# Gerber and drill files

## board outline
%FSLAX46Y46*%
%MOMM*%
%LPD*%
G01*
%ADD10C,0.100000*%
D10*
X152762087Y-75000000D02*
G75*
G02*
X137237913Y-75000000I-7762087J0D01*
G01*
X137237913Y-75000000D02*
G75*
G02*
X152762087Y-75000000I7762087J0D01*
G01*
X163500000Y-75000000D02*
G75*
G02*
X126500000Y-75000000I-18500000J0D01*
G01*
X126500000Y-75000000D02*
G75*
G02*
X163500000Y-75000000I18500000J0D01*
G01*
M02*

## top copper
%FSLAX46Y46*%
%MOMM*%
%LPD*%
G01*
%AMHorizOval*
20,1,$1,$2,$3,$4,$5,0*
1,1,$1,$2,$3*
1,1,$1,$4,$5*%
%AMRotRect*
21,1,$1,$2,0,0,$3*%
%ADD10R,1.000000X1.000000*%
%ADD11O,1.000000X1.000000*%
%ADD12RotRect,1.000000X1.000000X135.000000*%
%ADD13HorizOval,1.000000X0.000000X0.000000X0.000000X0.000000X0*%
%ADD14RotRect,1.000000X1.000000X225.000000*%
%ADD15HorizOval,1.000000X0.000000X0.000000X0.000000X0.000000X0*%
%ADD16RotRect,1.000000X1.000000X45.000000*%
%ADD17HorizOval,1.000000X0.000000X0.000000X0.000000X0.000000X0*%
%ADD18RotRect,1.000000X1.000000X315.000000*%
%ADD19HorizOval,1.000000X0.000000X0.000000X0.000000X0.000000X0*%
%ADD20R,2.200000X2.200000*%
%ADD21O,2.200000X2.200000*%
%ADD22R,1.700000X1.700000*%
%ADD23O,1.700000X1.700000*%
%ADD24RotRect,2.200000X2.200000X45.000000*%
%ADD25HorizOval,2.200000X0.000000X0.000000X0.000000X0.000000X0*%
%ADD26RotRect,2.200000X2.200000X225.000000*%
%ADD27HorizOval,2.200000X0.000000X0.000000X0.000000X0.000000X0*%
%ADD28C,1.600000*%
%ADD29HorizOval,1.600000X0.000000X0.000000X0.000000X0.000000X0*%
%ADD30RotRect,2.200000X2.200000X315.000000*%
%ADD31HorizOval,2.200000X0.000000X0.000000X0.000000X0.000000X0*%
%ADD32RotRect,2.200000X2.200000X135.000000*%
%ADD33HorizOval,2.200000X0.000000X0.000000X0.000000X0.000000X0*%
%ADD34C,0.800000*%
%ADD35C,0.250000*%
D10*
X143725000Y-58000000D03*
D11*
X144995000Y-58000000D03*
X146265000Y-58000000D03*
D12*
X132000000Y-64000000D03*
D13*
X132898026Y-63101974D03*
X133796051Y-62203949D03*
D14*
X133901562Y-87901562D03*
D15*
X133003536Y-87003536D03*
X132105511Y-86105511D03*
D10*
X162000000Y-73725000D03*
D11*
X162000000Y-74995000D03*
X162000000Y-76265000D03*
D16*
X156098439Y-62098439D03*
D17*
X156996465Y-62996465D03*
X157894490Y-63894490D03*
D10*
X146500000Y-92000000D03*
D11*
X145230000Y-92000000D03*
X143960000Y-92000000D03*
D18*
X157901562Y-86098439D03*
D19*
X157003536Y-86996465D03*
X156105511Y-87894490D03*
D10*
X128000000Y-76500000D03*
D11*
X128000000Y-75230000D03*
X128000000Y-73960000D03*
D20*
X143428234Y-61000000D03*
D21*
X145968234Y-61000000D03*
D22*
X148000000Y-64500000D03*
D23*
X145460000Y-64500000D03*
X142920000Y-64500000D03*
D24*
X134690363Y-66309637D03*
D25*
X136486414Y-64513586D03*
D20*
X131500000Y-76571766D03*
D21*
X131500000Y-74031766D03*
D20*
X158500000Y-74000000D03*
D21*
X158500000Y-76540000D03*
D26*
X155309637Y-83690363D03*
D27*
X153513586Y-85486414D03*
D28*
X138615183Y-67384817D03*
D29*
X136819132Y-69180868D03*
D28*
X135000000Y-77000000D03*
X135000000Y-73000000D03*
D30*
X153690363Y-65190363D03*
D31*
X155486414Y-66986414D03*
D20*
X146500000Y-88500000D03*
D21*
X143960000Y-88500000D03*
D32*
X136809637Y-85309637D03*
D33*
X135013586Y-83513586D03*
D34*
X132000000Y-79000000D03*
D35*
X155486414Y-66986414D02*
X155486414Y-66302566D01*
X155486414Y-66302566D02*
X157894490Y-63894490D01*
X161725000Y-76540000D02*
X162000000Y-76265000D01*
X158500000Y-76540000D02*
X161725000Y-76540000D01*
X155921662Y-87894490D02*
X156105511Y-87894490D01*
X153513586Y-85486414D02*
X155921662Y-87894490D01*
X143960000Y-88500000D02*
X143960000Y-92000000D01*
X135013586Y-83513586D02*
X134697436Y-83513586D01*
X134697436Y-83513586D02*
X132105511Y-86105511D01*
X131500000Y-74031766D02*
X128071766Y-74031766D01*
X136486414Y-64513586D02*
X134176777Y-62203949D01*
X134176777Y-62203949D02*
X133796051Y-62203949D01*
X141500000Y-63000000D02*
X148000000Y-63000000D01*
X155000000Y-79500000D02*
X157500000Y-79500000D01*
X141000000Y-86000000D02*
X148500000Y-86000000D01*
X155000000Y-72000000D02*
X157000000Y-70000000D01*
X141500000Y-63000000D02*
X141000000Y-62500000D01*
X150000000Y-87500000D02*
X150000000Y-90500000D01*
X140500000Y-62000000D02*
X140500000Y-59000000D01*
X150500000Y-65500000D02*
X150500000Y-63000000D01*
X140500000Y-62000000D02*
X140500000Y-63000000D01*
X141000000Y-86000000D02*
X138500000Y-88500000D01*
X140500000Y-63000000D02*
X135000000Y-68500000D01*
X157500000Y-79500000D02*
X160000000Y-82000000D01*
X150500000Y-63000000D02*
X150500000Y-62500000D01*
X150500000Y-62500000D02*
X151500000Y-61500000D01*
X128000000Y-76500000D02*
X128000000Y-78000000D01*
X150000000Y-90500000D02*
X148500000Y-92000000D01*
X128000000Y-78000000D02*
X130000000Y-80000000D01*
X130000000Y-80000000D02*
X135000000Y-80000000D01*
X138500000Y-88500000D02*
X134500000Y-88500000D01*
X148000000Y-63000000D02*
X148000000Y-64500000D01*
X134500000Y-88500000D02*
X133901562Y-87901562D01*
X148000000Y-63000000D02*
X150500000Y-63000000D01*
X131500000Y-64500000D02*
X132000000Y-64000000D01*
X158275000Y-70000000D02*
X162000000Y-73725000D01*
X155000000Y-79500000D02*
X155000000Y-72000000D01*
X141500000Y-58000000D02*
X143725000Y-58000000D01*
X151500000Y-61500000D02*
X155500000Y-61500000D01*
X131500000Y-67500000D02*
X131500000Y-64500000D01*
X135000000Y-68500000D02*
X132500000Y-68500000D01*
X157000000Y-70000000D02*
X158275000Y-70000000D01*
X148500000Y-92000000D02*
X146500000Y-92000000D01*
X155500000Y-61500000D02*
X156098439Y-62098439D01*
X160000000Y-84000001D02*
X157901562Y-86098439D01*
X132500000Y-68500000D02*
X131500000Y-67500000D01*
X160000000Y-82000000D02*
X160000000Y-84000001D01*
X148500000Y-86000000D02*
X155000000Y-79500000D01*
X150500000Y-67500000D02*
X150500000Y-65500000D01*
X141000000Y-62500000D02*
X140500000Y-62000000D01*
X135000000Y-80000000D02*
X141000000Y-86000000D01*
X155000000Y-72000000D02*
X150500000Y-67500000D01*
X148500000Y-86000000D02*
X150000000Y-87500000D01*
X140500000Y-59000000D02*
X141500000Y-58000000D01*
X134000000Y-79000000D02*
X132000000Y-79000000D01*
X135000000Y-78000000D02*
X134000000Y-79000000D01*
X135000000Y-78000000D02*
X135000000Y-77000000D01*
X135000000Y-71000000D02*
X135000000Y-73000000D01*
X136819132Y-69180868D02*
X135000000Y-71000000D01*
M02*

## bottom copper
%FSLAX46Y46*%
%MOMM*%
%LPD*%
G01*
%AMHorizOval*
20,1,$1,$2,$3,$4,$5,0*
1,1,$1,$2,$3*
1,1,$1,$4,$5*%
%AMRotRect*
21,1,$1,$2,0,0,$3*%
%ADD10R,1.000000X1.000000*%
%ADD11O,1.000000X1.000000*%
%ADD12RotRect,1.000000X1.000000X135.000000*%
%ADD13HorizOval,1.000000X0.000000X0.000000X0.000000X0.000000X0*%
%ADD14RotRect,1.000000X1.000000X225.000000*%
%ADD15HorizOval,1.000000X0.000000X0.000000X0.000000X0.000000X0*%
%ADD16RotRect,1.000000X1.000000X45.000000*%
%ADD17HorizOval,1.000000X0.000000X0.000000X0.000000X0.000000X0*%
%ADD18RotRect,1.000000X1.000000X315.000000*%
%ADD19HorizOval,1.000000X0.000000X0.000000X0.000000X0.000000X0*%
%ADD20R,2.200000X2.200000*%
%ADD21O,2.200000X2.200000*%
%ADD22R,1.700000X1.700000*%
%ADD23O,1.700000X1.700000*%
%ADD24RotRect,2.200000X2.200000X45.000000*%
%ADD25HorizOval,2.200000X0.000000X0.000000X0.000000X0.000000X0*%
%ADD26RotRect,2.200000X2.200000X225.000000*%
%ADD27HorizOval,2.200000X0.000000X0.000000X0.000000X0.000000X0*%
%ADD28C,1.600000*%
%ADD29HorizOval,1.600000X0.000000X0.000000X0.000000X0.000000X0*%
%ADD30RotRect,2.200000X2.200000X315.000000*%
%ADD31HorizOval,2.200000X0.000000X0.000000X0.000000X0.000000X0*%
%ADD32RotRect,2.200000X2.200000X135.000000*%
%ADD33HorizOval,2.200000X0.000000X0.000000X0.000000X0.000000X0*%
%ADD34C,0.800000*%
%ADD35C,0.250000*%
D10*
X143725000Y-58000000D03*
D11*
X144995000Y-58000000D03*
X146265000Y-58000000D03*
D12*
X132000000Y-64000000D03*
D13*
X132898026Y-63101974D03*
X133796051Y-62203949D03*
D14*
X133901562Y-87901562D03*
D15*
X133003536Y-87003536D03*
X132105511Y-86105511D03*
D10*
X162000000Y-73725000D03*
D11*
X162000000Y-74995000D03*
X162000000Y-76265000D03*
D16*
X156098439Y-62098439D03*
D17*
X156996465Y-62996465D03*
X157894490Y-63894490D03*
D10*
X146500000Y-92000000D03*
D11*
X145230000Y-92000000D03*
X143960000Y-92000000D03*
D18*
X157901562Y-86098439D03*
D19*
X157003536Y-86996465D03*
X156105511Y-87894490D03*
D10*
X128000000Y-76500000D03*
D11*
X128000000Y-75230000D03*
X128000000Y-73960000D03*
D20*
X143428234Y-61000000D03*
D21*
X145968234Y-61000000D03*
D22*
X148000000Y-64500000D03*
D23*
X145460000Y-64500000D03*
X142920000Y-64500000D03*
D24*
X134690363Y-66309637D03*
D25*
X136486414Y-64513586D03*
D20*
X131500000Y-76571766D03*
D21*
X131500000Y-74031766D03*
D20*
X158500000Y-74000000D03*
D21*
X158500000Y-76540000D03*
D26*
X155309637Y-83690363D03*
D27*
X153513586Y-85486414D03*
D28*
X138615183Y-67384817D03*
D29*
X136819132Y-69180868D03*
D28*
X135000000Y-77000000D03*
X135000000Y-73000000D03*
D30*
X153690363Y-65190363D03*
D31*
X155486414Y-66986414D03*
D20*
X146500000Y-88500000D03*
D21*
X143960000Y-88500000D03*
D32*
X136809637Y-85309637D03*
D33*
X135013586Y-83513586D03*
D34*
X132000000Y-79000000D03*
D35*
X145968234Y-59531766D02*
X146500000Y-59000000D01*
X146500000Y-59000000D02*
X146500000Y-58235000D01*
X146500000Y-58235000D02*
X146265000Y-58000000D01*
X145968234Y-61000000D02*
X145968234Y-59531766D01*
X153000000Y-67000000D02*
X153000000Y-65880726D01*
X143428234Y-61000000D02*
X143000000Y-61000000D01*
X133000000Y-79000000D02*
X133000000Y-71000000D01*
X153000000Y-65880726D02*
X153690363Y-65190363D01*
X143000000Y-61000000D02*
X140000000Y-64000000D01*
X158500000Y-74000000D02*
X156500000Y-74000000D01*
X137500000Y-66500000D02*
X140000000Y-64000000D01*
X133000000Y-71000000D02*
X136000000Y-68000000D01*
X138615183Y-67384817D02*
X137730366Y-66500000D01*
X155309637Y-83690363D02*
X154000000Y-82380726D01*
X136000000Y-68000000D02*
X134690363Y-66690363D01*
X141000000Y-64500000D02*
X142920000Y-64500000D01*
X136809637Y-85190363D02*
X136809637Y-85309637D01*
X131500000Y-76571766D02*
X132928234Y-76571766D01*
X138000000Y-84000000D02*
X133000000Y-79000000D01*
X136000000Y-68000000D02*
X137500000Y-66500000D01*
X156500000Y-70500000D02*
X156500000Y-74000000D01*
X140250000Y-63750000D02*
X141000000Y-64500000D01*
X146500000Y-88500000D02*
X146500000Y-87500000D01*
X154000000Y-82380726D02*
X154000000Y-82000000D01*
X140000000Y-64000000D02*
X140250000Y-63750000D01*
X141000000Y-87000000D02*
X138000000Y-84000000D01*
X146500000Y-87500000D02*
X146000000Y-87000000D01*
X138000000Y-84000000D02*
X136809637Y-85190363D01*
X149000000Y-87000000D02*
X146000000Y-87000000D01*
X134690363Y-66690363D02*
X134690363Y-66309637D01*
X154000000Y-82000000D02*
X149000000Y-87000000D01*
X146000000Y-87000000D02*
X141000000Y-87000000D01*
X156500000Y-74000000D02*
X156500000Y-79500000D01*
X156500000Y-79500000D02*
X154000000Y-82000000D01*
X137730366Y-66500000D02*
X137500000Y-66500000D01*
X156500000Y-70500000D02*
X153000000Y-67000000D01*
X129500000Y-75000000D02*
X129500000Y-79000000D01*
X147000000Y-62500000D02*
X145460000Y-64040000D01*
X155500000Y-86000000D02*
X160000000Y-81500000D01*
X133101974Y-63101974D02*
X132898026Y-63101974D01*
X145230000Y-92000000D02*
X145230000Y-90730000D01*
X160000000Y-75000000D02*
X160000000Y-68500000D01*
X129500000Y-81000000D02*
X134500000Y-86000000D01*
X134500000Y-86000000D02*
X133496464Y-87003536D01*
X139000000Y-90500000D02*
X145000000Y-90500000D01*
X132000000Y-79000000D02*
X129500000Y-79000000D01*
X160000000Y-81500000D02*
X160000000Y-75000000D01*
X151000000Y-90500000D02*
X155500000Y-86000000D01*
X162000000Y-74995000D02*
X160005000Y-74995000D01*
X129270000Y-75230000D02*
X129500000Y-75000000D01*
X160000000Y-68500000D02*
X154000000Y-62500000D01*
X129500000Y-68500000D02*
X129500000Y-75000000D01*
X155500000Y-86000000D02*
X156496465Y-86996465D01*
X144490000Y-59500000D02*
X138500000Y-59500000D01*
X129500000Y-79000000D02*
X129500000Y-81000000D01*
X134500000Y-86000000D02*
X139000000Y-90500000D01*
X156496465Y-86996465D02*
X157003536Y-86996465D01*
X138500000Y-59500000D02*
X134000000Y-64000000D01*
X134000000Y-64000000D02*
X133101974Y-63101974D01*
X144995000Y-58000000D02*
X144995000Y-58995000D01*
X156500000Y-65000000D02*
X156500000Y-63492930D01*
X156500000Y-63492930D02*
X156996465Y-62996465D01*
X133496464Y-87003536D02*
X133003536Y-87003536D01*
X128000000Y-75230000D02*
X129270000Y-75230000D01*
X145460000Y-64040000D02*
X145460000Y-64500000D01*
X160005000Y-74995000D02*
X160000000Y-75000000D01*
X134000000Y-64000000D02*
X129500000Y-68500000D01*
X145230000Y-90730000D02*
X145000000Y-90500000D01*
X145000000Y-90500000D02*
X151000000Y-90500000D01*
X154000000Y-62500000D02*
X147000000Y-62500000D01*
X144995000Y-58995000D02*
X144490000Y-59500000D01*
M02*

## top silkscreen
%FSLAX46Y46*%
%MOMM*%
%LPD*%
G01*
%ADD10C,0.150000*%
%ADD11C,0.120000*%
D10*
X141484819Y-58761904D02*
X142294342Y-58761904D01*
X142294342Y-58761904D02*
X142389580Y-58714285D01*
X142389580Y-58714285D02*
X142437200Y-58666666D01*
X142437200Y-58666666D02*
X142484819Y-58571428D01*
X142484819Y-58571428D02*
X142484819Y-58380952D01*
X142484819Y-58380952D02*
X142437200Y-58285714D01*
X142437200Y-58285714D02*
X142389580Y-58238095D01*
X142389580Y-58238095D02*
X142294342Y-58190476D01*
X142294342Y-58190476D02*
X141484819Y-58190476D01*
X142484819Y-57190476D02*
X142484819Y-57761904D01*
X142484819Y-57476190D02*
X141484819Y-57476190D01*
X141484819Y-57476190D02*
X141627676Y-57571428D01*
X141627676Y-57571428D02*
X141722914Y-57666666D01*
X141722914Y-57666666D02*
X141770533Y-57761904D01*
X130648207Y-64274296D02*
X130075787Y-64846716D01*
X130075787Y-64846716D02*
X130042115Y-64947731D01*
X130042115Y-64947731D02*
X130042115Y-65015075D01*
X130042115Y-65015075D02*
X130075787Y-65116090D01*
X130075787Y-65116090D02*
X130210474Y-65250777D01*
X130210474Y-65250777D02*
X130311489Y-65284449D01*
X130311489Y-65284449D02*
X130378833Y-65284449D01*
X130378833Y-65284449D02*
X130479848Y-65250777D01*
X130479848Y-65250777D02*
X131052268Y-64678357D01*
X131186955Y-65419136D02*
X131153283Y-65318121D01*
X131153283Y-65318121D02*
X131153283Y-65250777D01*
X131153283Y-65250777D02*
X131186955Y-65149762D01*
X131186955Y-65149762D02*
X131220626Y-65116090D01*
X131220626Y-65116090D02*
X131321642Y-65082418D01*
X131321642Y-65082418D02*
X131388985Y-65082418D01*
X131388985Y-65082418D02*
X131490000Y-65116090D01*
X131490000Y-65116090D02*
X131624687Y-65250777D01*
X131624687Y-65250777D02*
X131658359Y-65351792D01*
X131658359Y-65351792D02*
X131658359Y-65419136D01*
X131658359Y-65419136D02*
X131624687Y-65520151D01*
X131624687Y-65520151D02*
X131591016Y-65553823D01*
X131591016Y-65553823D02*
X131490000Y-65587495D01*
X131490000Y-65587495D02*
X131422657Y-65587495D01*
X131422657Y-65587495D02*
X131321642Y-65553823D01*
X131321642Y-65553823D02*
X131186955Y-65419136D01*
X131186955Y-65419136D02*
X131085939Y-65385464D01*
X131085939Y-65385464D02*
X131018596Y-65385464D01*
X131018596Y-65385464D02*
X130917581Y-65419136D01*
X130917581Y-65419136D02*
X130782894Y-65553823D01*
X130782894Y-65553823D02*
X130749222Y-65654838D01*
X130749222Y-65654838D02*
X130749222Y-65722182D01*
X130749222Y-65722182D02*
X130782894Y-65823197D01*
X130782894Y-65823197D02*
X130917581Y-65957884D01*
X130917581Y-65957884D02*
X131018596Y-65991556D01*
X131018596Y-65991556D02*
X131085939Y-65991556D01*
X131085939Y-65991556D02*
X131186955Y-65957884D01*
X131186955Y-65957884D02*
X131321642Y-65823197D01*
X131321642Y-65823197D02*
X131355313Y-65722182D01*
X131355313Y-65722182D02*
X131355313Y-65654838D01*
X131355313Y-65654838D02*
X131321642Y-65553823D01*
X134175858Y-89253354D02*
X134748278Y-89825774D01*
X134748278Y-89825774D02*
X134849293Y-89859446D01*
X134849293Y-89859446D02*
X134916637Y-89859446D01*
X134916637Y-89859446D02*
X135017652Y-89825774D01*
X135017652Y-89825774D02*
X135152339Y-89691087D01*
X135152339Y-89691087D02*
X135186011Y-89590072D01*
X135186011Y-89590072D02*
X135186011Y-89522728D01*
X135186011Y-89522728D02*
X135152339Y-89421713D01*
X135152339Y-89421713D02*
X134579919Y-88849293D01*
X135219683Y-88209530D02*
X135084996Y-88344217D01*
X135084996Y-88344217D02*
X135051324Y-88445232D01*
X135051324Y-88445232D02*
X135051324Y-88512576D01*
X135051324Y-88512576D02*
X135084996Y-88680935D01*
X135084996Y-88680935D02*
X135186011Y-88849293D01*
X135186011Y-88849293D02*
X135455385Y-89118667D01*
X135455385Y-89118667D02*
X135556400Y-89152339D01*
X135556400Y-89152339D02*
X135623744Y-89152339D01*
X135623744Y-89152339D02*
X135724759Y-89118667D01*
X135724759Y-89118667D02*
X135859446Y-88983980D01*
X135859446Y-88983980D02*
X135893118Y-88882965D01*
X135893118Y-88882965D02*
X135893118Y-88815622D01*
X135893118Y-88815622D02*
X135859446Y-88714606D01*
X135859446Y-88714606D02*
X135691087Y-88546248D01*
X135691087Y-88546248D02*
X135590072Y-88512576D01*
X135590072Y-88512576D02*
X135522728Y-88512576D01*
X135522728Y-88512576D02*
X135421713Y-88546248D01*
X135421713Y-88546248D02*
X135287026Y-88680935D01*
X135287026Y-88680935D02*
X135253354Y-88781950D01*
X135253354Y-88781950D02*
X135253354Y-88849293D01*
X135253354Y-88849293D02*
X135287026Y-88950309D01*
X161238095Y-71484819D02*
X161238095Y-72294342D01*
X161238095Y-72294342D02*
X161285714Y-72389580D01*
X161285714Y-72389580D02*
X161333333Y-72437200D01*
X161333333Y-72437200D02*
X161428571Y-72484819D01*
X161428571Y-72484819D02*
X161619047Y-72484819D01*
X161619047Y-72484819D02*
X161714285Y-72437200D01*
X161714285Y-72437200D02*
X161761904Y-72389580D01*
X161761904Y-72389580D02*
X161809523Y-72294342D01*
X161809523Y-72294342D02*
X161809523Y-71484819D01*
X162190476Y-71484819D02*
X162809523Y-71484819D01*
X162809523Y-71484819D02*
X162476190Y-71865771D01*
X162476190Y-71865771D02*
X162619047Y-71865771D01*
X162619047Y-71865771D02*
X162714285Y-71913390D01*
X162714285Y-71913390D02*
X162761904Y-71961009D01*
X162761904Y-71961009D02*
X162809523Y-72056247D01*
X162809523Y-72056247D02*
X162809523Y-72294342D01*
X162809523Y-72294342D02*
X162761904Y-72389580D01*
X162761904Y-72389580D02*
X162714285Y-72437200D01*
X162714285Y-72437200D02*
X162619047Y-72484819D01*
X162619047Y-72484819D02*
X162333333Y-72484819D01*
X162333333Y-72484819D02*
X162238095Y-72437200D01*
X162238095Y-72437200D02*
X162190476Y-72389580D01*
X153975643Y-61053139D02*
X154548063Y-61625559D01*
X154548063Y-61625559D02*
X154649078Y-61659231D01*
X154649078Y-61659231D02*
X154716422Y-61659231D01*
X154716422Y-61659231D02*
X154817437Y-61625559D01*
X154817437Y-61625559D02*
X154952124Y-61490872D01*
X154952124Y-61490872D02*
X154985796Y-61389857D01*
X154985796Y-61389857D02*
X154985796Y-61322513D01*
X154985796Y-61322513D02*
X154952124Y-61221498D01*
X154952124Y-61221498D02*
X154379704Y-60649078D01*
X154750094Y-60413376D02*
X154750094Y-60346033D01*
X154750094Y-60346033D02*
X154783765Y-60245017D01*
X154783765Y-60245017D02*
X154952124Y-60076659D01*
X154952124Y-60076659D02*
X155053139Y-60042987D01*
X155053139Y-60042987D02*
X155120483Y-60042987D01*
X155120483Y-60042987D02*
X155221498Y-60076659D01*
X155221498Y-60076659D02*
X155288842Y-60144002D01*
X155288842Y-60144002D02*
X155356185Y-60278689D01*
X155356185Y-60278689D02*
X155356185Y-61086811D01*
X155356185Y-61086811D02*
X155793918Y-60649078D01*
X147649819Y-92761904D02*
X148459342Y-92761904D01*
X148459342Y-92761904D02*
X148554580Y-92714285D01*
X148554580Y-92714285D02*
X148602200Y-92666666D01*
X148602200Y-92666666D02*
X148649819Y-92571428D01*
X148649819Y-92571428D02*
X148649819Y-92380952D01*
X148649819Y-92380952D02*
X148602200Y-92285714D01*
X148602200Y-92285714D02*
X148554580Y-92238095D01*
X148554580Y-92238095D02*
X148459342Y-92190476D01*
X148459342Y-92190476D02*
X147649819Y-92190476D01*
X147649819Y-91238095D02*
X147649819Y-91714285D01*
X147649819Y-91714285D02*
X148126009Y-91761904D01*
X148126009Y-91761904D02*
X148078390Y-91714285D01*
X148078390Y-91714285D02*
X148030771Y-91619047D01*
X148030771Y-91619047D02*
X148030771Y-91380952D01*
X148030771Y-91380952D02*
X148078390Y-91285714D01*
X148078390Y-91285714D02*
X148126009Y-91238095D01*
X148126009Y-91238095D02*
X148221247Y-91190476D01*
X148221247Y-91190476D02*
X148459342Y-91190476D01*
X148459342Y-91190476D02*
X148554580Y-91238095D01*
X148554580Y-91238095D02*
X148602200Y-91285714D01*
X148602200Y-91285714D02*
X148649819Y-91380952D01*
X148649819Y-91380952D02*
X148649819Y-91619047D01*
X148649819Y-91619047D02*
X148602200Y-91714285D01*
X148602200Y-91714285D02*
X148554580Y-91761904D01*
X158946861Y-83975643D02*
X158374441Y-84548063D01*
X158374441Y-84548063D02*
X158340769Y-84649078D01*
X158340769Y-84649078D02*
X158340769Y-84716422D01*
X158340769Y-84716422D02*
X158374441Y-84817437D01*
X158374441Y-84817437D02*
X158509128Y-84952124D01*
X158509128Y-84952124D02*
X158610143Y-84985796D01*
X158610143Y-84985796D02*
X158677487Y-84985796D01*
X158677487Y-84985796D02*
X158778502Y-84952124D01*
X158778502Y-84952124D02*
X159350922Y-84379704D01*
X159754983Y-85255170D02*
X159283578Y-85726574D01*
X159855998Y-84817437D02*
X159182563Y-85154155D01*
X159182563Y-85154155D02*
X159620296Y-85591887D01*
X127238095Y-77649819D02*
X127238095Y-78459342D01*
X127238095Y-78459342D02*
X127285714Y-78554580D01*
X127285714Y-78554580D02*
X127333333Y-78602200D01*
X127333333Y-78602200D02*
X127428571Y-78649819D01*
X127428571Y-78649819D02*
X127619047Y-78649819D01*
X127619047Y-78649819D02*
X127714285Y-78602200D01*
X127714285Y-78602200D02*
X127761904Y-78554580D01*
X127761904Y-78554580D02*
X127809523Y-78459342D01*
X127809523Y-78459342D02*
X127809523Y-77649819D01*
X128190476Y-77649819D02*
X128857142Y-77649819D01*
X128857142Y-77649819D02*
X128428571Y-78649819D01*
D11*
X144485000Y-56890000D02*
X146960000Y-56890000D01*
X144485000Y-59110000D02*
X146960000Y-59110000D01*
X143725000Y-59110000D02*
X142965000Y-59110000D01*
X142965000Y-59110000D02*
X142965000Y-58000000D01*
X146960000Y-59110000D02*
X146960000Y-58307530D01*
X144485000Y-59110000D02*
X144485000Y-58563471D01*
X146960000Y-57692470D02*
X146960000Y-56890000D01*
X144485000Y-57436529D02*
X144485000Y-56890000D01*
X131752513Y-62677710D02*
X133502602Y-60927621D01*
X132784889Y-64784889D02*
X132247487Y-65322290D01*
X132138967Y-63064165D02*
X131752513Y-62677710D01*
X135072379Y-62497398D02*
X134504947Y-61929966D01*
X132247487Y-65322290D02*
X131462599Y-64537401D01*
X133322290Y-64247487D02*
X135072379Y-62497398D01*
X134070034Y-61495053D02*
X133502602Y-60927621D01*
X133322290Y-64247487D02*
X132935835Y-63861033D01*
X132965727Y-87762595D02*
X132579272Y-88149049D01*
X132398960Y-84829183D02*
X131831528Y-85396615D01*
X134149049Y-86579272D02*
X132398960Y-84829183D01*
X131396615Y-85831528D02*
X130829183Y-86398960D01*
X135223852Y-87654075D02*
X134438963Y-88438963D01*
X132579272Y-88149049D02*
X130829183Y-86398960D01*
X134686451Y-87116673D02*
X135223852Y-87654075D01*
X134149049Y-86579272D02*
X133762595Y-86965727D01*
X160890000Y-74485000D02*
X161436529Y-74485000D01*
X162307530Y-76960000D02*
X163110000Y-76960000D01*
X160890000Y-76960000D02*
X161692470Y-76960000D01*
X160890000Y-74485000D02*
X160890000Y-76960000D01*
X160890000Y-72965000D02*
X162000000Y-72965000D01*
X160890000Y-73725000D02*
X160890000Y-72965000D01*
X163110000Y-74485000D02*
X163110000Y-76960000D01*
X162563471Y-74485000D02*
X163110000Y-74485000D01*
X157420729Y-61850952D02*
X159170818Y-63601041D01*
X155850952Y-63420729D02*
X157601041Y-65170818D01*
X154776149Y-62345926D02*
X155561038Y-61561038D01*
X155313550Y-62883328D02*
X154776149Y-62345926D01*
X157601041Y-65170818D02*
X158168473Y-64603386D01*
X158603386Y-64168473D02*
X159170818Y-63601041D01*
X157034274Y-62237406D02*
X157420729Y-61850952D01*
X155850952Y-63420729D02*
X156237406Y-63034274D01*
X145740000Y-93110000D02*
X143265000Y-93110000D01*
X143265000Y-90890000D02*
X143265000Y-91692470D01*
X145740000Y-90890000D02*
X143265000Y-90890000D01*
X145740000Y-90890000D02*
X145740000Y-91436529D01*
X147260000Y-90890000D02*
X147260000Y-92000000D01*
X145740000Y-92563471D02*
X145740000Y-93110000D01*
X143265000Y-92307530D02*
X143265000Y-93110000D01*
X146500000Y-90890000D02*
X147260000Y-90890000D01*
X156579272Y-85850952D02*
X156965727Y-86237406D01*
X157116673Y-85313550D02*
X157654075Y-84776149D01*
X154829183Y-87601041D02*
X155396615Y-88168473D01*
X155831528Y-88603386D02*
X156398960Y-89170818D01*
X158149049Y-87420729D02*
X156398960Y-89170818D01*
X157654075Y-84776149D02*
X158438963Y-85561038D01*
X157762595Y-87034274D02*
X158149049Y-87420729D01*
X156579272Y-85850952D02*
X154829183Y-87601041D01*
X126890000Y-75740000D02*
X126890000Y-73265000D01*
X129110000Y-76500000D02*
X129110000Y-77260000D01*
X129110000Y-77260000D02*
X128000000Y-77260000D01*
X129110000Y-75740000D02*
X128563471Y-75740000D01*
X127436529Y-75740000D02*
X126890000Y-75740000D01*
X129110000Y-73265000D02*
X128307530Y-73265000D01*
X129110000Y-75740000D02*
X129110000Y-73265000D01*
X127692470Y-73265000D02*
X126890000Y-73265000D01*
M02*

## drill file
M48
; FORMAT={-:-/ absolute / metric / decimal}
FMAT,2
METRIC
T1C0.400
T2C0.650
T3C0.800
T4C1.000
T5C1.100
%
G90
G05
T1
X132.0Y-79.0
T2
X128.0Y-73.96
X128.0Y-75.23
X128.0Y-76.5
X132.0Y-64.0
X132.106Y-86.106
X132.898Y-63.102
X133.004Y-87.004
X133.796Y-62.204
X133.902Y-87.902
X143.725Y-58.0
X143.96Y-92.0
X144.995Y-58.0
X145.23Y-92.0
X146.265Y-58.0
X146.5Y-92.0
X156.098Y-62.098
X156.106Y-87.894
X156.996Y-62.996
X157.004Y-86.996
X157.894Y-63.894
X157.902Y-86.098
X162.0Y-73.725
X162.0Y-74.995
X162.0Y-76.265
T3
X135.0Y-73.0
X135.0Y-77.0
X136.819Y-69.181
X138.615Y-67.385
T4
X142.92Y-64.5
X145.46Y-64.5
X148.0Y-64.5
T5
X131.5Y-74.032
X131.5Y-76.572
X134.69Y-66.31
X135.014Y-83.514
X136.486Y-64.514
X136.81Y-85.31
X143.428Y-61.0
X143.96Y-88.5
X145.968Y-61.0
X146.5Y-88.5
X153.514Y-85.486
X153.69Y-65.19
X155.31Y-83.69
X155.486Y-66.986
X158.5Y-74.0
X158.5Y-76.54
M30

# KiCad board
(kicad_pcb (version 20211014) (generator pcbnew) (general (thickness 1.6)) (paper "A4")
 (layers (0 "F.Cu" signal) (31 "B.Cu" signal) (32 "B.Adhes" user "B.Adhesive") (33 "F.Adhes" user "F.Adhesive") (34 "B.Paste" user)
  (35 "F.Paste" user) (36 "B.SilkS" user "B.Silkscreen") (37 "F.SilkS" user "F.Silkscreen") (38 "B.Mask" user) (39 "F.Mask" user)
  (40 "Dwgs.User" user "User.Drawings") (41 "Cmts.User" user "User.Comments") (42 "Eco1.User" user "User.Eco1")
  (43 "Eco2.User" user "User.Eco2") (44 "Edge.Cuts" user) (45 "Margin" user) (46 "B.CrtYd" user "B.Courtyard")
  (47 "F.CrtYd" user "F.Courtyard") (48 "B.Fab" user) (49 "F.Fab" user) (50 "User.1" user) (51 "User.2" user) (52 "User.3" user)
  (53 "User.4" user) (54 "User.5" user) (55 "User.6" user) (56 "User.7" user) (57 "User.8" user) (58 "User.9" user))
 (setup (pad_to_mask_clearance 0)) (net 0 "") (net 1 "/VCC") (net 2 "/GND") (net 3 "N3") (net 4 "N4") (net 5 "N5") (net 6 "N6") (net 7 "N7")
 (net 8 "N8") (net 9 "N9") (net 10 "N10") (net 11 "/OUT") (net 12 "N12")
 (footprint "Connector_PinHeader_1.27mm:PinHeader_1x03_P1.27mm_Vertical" (layer "F.Cu") (at 143.725 58 90)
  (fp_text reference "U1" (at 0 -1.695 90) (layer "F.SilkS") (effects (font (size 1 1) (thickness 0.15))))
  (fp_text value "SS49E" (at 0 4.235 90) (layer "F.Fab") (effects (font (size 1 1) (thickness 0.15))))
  (fp_line (start 1.11 0.76) (end 1.11 3.235) (layer "F.SilkS") (width 0.12))
  (fp_line (start -1.11 0.76) (end -1.11 3.235) (layer "F.SilkS") (width 0.12))
  (fp_line (start -1.11 0) (end -1.11 -0.76) (layer "F.SilkS") (width 0.12))
  (fp_line (start -1.11 -0.76) (end 0 -0.76) (layer "F.SilkS") (width 0.12))
  (fp_line (start -1.11 3.235) (end -0.30753 3.235) (layer "F.SilkS") (width 0.12))
  (fp_line (start -1.11 0.76) (end -0.563471 0.76) (layer "F.SilkS") (width 0.12))
  (fp_line (start 0.30753 3.235) (end 1.11 3.235) (layer "F.SilkS") (width 0.12))
  (fp_line (start 0.563471 0.76) (end 1.11 0.76) (layer "F.SilkS") (width 0.12))
  (pad "1" thru_hole rect locked (at 0 0 90) (size 1 1) (drill 0.65) (layers *.Cu *.Mask) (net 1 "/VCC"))
  (pad "2" thru_hole oval locked (at 0 1.27 90) (size 1 1) (drill 0.65) (layers *.Cu *.Mask) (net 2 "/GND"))
  (pad "3" thru_hole oval locked (at 0 2.54 90) (size 1 1) (drill 0.65) (layers *.Cu *.Mask) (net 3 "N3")))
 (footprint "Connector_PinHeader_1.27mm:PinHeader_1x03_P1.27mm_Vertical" (layer "F.Cu") (at 132 64 135)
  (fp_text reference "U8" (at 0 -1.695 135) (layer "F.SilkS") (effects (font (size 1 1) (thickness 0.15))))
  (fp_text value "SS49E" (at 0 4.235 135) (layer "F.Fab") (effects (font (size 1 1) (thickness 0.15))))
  (fp_line (start 1.11 0.76) (end 1.11 3.235) (layer "F.SilkS") (width 0.12))
  (fp_line (start -1.11 0) (end -1.11 -0.76) (layer "F.SilkS") (width 0.12))
  (fp_line (start 0.563471 0.76) (end 1.11 0.76) (layer "F.SilkS") (width 0.12))
  (fp_line (start -1.11 3.235) (end -0.30753 3.235) (layer "F.SilkS") (width 0.12))
  (fp_line (start -1.11 -0.76) (end 0 -0.76) (layer "F.SilkS") (width 0.12))
  (fp_line (start -1.11 0.76) (end -1.11 3.235) (layer "F.SilkS") (width 0.12))
  (fp_line (start 0.30753 3.235) (end 1.11 3.235) (layer "F.SilkS") (width 0.12))
  (fp_line (start -1.11 0.76) (end -0.563471 0.76) (layer "F.SilkS") (width 0.12))
  (pad "1" thru_hole rect locked (at 0 0 135) (size 1 1) (drill 0.65) (layers *.Cu *.Mask) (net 1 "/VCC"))
  (pad "2" thru_hole oval locked (at 0 1.27 135) (size 1 1) (drill 0.65) (layers *.Cu *.Mask) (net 2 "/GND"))
  (pad "3" thru_hole oval locked (at 0 2.54 135) (size 1 1) (drill 0.65) (layers *.Cu *.Mask) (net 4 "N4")))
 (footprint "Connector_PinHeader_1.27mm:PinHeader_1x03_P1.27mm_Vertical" (layer "F.Cu") (at 133.901562 87.901562 -135)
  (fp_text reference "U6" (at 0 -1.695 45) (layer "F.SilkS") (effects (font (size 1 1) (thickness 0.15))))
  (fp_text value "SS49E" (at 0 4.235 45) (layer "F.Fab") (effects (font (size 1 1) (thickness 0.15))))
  (fp_line (start 0.563471 0.76) (end 1.11 0.76) (layer "F.SilkS") (width 0.12))
  (fp_line (start -1.11 3.235) (end -0.30753 3.235) (layer "F.SilkS") (width 0.12))
  (fp_line (start -1.11 0.76) (end -1.11 3.235) (layer "F.SilkS") (width 0.12))
  (fp_line (start 0.30753 3.235) (end 1.11 3.235) (layer "F.SilkS") (width 0.12))
  (fp_line (start -1.11 -0.76) (end 0 -0.76) (layer "F.SilkS") (width 0.12))
  (fp_line (start 1.11 0.76) (end 1.11 3.235) (layer "F.SilkS") (width 0.12))
  (fp_line (start -1.11 0) (end -1.11 -0.76) (layer "F.SilkS") (width 0.12))
  (fp_line (start -1.11 0.76) (end -0.563471 0.76) (layer "F.SilkS") (width 0.12))
  (pad "1" thru_hole rect locked (at 0 0 225) (size 1 1) (drill 0.65) (layers *.Cu *.Mask) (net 1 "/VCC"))
  (pad "2" thru_hole oval locked (at 0 1.27 225) (size 1 1) (drill 0.65) (layers *.Cu *.Mask) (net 2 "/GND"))
  (pad "3" thru_hole oval locked (at 0 2.54 225) (size 1 1) (drill 0.65) (layers *.Cu *.Mask) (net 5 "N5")))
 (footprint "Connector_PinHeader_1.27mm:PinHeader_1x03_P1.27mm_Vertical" (layer "F.Cu") (at 162 73.725)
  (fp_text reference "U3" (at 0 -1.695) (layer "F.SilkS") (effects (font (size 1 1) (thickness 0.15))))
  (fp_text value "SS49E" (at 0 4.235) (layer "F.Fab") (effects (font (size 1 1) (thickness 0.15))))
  (fp_line (start -1.11 0.76) (end -0.563471 0.76) (layer "F.SilkS") (width 0.12))
  (fp_line (start 0.30753 3.235) (end 1.11 3.235) (layer "F.SilkS") (width 0.12))
  (fp_line (start -1.11 3.235) (end -0.30753 3.235) (layer "F.SilkS") (width 0.12))
  (fp_line (start -1.11 0.76) (end -1.11 3.235) (layer "F.SilkS") (width 0.12))
  (fp_line (start -1.11 -0.76) (end 0 -0.76) (layer "F.SilkS") (width 0.12))
  (fp_line (start -1.11 0) (end -1.11 -0.76) (layer "F.SilkS") (width 0.12))
  (fp_line (start 1.11 0.76) (end 1.11 3.235) (layer "F.SilkS") (width 0.12))
  (fp_line (start 0.563471 0.76) (end 1.11 0.76) (layer "F.SilkS") (width 0.12))
  (pad "1" thru_hole rect locked (at 0 0) (size 1 1) (drill 0.65) (layers *.Cu *.Mask) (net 1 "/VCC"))
  (pad "2" thru_hole oval locked (at 0 1.27) (size 1 1) (drill 0.65) (layers *.Cu *.Mask) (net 2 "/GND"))
  (pad "3" thru_hole oval locked (at 0 2.54) (size 1 1) (drill 0.65) (layers *.Cu *.Mask) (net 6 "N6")))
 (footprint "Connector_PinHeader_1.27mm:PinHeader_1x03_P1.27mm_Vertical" (layer "F.Cu") (at 156.098439 62.098439 45)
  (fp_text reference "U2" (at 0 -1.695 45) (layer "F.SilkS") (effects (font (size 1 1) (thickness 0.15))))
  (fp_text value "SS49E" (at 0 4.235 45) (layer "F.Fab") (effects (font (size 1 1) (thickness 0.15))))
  (fp_line (start 1.11 0.76) (end 1.11 3.235) (layer "F.SilkS") (width 0.12))
  (fp_line (start -1.11 0.76) (end -1.11 3.235) (layer "F.SilkS") (width 0.12))
  (fp_line (start -1.11 -0.76) (end 0 -0.76) (layer "F.SilkS") (width 0.12))
  (fp_line (start -1.11 0) (end -1.11 -0.76) (layer "F.SilkS") (width 0.12))
  (fp_line (start -1.11 3.235) (end -0.30753 3.235) (layer "F.SilkS") (width 0.12))
  (fp_line (start 0.30753 3.235) (end 1.11 3.235) (layer "F.SilkS") (width 0.12))
  (fp_line (start 0.563471 0.76) (end 1.11 0.76) (layer "F.SilkS") (width 0.12))
  (fp_line (start -1.11 0.76) (end -0.563471 0.76) (layer "F.SilkS") (width 0.12))
  (pad "1" thru_hole rect locked (at 0 0 45) (size 1 1) (drill 0.65) (layers *.Cu *.Mask) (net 1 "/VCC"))
  (pad "2" thru_hole oval locked (at 0 1.27 45) (size 1 1) (drill 0.65) (layers *.Cu *.Mask) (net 2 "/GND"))
  (pad "3" thru_hole oval locked (at 0 2.54 45) (size 1 1) (drill 0.65) (layers *.Cu *.Mask) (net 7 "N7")))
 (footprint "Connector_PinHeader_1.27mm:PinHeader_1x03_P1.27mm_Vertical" (layer "F.Cu") (at 146.5 92 -90)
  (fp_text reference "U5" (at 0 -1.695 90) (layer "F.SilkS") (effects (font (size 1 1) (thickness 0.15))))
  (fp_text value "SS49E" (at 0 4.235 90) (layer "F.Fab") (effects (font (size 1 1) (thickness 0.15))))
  (fp_line (start 1.11 0.76) (end 1.11 3.235) (layer "F.SilkS") (width 0.12))
  (fp_line (start -1.11 3.235) (end -0.30753 3.235) (layer "F.SilkS") (width 0.12))
  (fp_line (start -1.11 0.76) (end -1.11 3.235) (layer "F.SilkS") (width 0.12))
  (fp_line (start -1.11 0.76) (end -0.563471 0.76) (layer "F.SilkS") (width 0.12))
  (fp_line (start -1.11 -0.76) (end 0 -0.76) (layer "F.SilkS") (width 0.12))
  (fp_line (start 0.563471 0.76) (end 1.11 0.76) (layer "F.SilkS") (width 0.12))
  (fp_line (start 0.30753 3.235) (end 1.11 3.235) (layer "F.SilkS") (width 0.12))
  (fp_line (start -1.11 0) (end -1.11 -0.76) (layer "F.SilkS") (width 0.12))
  (pad "1" thru_hole rect locked (at 0 0 270) (size 1 1) (drill 0.65) (layers *.Cu *.Mask) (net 1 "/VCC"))
  (pad "2" thru_hole oval locked (at 0 1.27 270) (size 1 1) (drill 0.65) (layers *.Cu *.Mask) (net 2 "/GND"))
  (pad "3" thru_hole oval locked (at 0 2.54 270) (size 1 1) (drill 0.65) (layers *.Cu *.Mask) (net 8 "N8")))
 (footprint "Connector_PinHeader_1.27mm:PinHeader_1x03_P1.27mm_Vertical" (layer "F.Cu") (at 157.901562 86.098439 -45)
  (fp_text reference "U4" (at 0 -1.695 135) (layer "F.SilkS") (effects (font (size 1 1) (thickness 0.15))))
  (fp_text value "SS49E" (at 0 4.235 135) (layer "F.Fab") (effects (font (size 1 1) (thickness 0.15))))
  (fp_line (start -1.11 0.76) (end -0.563471 0.76) (layer "F.SilkS") (width 0.12))
  (fp_line (start -1.11 0) (end -1.11 -0.76) (layer "F.SilkS") (width 0.12))
  (fp_line (start -1.11 3.235) (end -0.30753 3.235) (layer "F.SilkS") (width 0.12))
  (fp_line (start 0.30753 3.235) (end 1.11 3.235) (layer "F.SilkS") (width 0.12))
  (fp_line (start 1.11 0.76) (end 1.11 3.235) (layer "F.SilkS") (width 0.12))
  (fp_line (start -1.11 -0.76) (end 0 -0.76) (layer "F.SilkS") (width 0.12))
  (fp_line (start 0.563471 0.76) (end 1.11 0.76) (layer "F.SilkS") (width 0.12))
  (fp_line (start -1.11 0.76) (end -1.11 3.235) (layer "F.SilkS") (width 0.12))
  (pad "1" thru_hole rect locked (at 0 0 315) (size 1 1) (drill 0.65) (layers *.Cu *.Mask) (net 1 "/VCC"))
  (pad "2" thru_hole oval locked (at 0 1.27 315) (size 1 1) (drill 0.65) (layers *.Cu *.Mask) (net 2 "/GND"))
  (pad "3" thru_hole oval locked (at 0 2.54 315) (size 1 1) (drill 0.65) (layers *.Cu *.Mask) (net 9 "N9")))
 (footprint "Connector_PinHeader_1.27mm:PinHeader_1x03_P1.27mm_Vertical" (layer "F.Cu") (at 128 76.5 180)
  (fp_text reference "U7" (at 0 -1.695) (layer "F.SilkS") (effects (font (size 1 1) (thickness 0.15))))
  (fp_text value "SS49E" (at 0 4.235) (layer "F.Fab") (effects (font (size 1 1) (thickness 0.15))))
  (fp_line (start 1.11 0.76) (end 1.11 3.235) (layer "F.SilkS") (width 0.12))
  (fp_line (start -1.11 0) (end -1.11 -0.76) (layer "F.SilkS") (width 0.12))
  (fp_line (start -1.11 -0.76) (end 0 -0.76) (layer "F.SilkS") (width 0.12))
  (fp_line (start -1.11 0.76) (end -0.563471 0.76) (layer "F.SilkS") (width 0.12))
  (fp_line (start 0.563471 0.76) (end 1.11 0.76) (layer "F.SilkS") (width 0.12))
  (fp_line (start -1.11 3.235) (end -0.30753 3.235) (layer "F.SilkS") (width 0.12))
  (fp_line (start -1.11 0.76) (end -1.11 3.235) (layer "F.SilkS") (width 0.12))
  (fp_line (start 0.30753 3.235) (end 1.11 3.235) (layer "F.SilkS") (width 0.12))
  (pad "1" thru_hole rect locked (at 0 0 180) (size 1 1) (drill 0.65) (layers *.Cu *.Mask) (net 1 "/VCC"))
  (pad "2" thru_hole oval locked (at 0 1.27 180) (size 1 1) (drill 0.65) (layers *.Cu *.Mask) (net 2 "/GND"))
  (pad "3" thru_hole oval locked (at 0 2.54 180) (size 1 1) (drill 0.65) (layers *.Cu *.Mask) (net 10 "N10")))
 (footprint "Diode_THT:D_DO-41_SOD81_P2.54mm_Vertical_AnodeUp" (layer "B.Cu") (at 143.428234 61)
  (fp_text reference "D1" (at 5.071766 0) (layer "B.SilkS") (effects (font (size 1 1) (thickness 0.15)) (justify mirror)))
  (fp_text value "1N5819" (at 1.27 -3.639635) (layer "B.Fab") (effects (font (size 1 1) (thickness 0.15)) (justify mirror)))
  (pad "1" thru_hole rect locked (at 0 0) (size 2.2 2.2) (drill 1.1) (layers *.Cu *.Mask) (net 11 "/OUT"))
  (pad "2" thru_hole oval locked (at 2.54 0) (size 2.2 2.2) (drill 1.1) (layers *.Cu *.Mask) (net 3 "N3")))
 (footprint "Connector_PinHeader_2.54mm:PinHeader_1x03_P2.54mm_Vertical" (layer "B.Cu") (at 148 64.5 90)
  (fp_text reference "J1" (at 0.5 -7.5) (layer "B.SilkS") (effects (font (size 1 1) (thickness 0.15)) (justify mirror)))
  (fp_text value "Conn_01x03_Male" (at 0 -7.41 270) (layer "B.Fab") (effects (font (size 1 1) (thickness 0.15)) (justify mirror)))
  (pad "1" thru_hole rect (at 0 0 90) (size 1.7 1.7) (drill 1) (layers *.Cu *.Mask) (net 1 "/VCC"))
  (pad "2" thru_hole oval (at 0 -2.54 90) (size 1.7 1.7) (drill 1) (layers *.Cu *.Mask) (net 2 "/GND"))
  (pad "3" thru_hole oval (at 0 -5.08 90) (size 1.7 1.7) (drill 1) (layers *.Cu *.Mask) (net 11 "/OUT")))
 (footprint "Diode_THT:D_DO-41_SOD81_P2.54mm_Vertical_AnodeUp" (layer "B.Cu") (at 134.690363 66.309637 45)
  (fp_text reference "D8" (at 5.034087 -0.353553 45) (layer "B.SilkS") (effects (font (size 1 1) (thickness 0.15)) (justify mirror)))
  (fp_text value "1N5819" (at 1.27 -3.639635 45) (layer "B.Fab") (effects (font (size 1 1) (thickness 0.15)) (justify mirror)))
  (pad "1" thru_hole rect locked (at 0 0 45) (size 2.2 2.2) (drill 1.1) (layers *.Cu *.Mask) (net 11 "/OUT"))
  (pad "2" thru_hole oval locked (at 2.54 0 45) (size 2.2 2.2) (drill 1.1) (layers *.Cu *.Mask) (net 4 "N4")))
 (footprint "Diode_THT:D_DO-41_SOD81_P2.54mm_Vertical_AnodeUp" (layer "B.Cu") (at 131.5 76.571766 90)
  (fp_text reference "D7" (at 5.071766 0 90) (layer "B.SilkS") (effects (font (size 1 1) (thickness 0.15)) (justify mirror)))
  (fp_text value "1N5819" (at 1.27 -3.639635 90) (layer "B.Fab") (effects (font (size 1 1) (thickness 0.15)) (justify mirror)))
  (pad "1" thru_hole rect locked (at 0 0 90) (size 2.2 2.2) (drill 1.1) (layers *.Cu *.Mask) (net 11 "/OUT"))
  (pad "2" thru_hole oval locked (at 2.54 0 90) (size 2.2 2.2) (drill 1.1) (layers *.Cu *.Mask) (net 10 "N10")))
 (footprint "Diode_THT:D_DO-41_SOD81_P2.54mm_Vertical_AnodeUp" (layer "B.Cu") (at 158.5 74 -90)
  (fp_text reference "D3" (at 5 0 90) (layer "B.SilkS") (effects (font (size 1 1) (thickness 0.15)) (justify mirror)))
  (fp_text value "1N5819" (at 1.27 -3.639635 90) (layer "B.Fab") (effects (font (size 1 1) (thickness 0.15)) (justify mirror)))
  (pad "1" thru_hole rect locked (at 0 0 270) (size 2.2 2.2) (drill 1.1) (layers *.Cu *.Mask) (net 11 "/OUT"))
  (pad "2" thru_hole oval locked (at 2.54 0 270) (size 2.2 2.2) (drill 1.1) (layers *.Cu *.Mask) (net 6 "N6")))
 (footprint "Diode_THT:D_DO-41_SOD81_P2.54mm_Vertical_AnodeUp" (layer "B.Cu") (at 155.309637 83.690363 -135)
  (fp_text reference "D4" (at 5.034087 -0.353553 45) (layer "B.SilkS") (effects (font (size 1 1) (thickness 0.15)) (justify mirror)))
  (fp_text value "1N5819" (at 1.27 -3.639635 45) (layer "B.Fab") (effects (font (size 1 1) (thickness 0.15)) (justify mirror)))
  (pad "1" thru_hole rect locked (at 0 0 225) (size 2.2 2.2) (drill 1.1) (layers *.Cu *.Mask) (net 11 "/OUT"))
  (pad "2" thru_hole oval locked (at 2.54 0 225) (size 2.2 2.2) (drill 1.1) (layers *.Cu *.Mask) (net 9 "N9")))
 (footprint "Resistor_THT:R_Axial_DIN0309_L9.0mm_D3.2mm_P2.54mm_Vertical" (layer "B.Cu") (at 138.615183 67.384817 -135)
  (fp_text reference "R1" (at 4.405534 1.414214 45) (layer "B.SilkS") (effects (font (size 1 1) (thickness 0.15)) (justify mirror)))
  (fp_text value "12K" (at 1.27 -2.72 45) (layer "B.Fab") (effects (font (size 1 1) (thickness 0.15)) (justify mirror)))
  (pad "1" thru_hole circle locked (at 0 0 225) (size 1.6 1.6) (drill 0.8) (layers *.Cu *.Mask) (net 11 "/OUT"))
  (pad "2" thru_hole oval locked (at 2.54 0 225) (size 1.6 1.6) (drill 0.8) (layers *.Cu *.Mask) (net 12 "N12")))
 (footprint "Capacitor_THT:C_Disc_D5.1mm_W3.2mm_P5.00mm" (layer "B.Cu") (at 135 77.5 90)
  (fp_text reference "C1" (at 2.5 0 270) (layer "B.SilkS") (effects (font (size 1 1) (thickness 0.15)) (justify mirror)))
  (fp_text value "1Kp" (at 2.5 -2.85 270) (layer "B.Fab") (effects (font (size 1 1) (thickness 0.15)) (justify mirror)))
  (pad "1" thru_hole circle (at 0.5 0 90) (size 1.6 1.6) (drill 0.8) (layers *.Cu *.Mask) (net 2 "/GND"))
  (pad "2" thru_hole circle (at 4.5 0 90) (size 1.6 1.6) (drill 0.8) (layers *.Cu *.Mask) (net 12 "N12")))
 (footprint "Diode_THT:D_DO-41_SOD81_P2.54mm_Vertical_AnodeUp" (layer "B.Cu") (at 153.690363 65.190363 -45)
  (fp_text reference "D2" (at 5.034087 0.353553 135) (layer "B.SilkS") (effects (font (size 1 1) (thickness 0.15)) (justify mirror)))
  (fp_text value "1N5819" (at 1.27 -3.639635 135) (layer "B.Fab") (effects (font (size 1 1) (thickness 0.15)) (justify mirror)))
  (pad "1" thru_hole rect locked (at 0 0 315) (size 2.2 2.2) (drill 1.1) (layers *.Cu *.Mask) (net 11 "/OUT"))
  (pad "2" thru_hole oval locked (at 2.54 0 315) (size 2.2 2.2) (drill 1.1) (layers *.Cu *.Mask) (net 7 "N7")))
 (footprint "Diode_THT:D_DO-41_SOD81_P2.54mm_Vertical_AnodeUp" (layer "B.Cu") (at 146.5 88.5 180)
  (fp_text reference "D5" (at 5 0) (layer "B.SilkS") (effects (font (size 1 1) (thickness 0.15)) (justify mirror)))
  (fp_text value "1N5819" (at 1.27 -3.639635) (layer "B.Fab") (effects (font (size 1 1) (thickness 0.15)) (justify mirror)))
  (pad "1" thru_hole rect locked (at 0 0 180) (size 2.2 2.2) (drill 1.1) (layers *.Cu *.Mask) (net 11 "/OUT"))
  (pad "2" thru_hole oval locked (at 2.54 0 180) (size 2.2 2.2) (drill 1.1) (layers *.Cu *.Mask) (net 8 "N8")))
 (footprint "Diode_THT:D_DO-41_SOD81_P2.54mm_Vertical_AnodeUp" (layer "B.Cu") (at 136.809637 85.309637 135)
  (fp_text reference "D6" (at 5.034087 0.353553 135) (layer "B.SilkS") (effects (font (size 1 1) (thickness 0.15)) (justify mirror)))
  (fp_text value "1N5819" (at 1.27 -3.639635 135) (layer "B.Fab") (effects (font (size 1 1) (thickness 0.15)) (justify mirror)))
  (pad "1" thru_hole rect locked (at 0 0 135) (size 2.2 2.2) (drill 1.1) (layers *.Cu *.Mask) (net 11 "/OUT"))
  (pad "2" thru_hole oval locked (at 2.54 0 135) (size 2.2 2.2) (drill 1.1) (layers *.Cu *.Mask) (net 5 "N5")))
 (gr_circle (center 145 75) (end 137.5 73) (layer "Edge.Cuts") (width 0.1) (fill none))
 (gr_circle (center 145 75) (end 163.5 75) (layer "Edge.Cuts") (width 0.1) (fill none))
 (segment (start 145.968234 59.531766) (end 146.5 59) (width 0.25) (layer "B.Cu") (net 3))
 (segment (start 146.5 59) (end 146.5 58.235) (width 0.25) (layer "B.Cu") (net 3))
 (segment (start 146.5 58.235) (end 146.265 58) (width 0.25) (layer "B.Cu") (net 3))
 (segment (start 145.968234 61) (end 145.968234 59.531766) (width 0.25) (layer "B.Cu") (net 3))
 (segment (start 155.486414 66.986414) (end 155.486414 66.302566) (width 0.25) (layer "F.Cu") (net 7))
 (segment (start 155.486414 66.302566) (end 157.89449 63.89449) (width 0.25) (layer "F.Cu") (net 7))
 (segment (start 161.725 76.54) (end 162 76.265) (width 0.25) (layer "F.Cu") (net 6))
 (segment (start 158.5 76.54) (end 161.725 76.54) (width 0.25) (layer "F.Cu") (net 6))
 (segment (start 155.921662 87.89449) (end 156.105511 87.89449) (width 0.25) (layer "F.Cu") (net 9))
 (segment (start 153.513586 85.486414) (end 155.921662 87.89449) (width 0.25) (layer "F.Cu") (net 9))
 (segment (start 143.96 88.5) (end 143.96 92) (width 0.25) (layer "F.Cu") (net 8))
 (segment (start 135.013586 83.513586) (end 134.697436 83.513586) (width 0.25) (layer "F.Cu") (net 5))
 (segment (start 134.697436 83.513586) (end 132.105511 86.105511) (width 0.25) (layer "F.Cu") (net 5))
 (segment (start 131.5 74.031766) (end 128.071766 74.031766) (width 0.25) (layer "F.Cu") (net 10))
 (segment (start 136.486414 64.513586) (end 134.176777 62.203949) (width 0.25) (layer "F.Cu") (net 4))
 (segment (start 134.176777 62.203949) (end 133.796051 62.203949) (width 0.25) (layer "F.Cu") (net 4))
 (segment (start 153 67) (end 153 65.880726) (width 0.25) (layer "B.Cu") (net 11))
 (segment (start 143.428234 61) (end 143 61) (width 0.25) (layer "B.Cu") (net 11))
 (segment (start 133 79) (end 133 71) (width 0.25) (layer "B.Cu") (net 11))
 (segment (start 153 65.880726) (end 153.690363 65.190363) (width 0.25) (layer "B.Cu") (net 11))
 (segment (start 143 61) (end 140 64) (width 0.25) (layer "B.Cu") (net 11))
 (segment (start 158.5 74) (end 156.5 74) (width 0.25) (layer "B.Cu") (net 11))
 (segment (start 137.5 66.5) (end 140 64) (width 0.25) (layer "B.Cu") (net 11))
 (segment (start 133 71) (end 136 68) (width 0.25) (layer "B.Cu") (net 11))
 (segment (start 138.615183 67.384817) (end 137.730366 66.5) (width 0.25) (layer "B.Cu") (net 11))
 (segment (start 155.309637 83.690363) (end 154 82.380726) (width 0.25) (layer "B.Cu") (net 11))
 (segment (start 136 68) (end 134.690363 66.690363) (width 0.25) (layer "B.Cu") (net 11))
 (segment (start 141 64.5) (end 142.92 64.5) (width 0.25) (layer "B.Cu") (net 11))
 (segment (start 136.809637 85.190363) (end 136.809637 85.309637) (width 0.25) (layer "B.Cu") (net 11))
 (segment (start 131.5 76.571766) (end 132.928234 76.571766) (width 0.25) (layer "B.Cu") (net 11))
 (segment (start 138 84) (end 133 79) (width 0.25) (layer "B.Cu") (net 11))
 (segment (start 136 68) (end 137.5 66.5) (width 0.25) (layer "B.Cu") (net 11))
 (segment (start 156.5 70.5) (end 156.5 74) (width 0.25) (layer "B.Cu") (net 11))
 (segment (start 140.25 63.75) (end 141 64.5) (width 0.25) (layer "B.Cu") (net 11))
 (segment (start 146.5 88.5) (end 146.5 87.5) (width 0.25) (layer "B.Cu") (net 11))
 (segment (start 154 82.380726) (end 154 82) (width 0.25) (layer "B.Cu") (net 11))
 (segment (start 140 64) (end 140.25 63.75) (width 0.25) (layer "B.Cu") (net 11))
 (segment (start 141 87) (end 138 84) (width 0.25) (layer "B.Cu") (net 11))
 (segment (start 146.5 87.5) (end 146 87) (width 0.25) (layer "B.Cu") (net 11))
 (segment (start 138 84) (end 136.809637 85.190363) (width 0.25) (layer "B.Cu") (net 11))
 (segment (start 149 87) (end 146 87) (width 0.25) (layer "B.Cu") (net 11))
 (segment (start 134.690363 66.690363) (end 134.690363 66.309637) (width 0.25) (layer "B.Cu") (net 11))
 (segment (start 154 82) (end 149 87) (width 0.25) (layer "B.Cu") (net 11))
 (segment (start 146 87) (end 141 87) (width 0.25) (layer "B.Cu") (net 11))
 (segment (start 156.5 74) (end 156.5 79.5) (width 0.25) (layer "B.Cu") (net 11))
 (segment (start 156.5 79.5) (end 154 82) (width 0.25) (layer "B.Cu") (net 11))
 (segment (start 137.730366 66.5) (end 137.5 66.5) (width 0.25) (layer "B.Cu") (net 11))
 (segment (start 156.5 70.5) (end 153 67) (width 0.25) (layer "B.Cu") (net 11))
 (segment (start 141.5 63) (end 148 63) (width 0.25) (layer "F.Cu") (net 1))
 (segment (start 155 79.5) (end 157.5 79.5) (width 0.25) (layer "F.Cu") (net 1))
 (segment (start 141 86) (end 148.5 86) (width 0.25) (layer "F.Cu") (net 1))
 (segment (start 155 72) (end 157 70) (width 0.25) (layer "F.Cu") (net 1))
 (segment (start 141.5 63) (end 141 62.5) (width 0.25) (layer "F.Cu") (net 1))
 (segment (start 150 87.5) (end 150 90.5) (width 0.25) (layer "F.Cu") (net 1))
 (segment (start 140.5 62) (end 140.5 59) (width 0.25) (layer "F.Cu") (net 1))
 (segment (start 150.5 65.5) (end 150.5 63) (width 0.25) (layer "F.Cu") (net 1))
 (segment (start 140.5 62) (end 140.5 63) (width 0.25) (layer "F.Cu") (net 1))
 (segment (start 141 86) (end 138.5 88.5) (width 0.25) (layer "F.Cu") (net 1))
 (segment (start 140.5 63) (end 135 68.5) (width 0.25) (layer "F.Cu") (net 1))
 (segment (start 157.5 79.5) (end 160 82) (width 0.25) (layer "F.Cu") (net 1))
 (segment (start 150.5 63) (end 150.5 62.5) (width 0.25) (layer "F.Cu") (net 1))
 (segment (start 150.5 62.5) (end 151.5 61.5) (width 0.25) (layer "F.Cu") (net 1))
 (segment (start 128 76.5) (end 128 78) (width 0.25) (layer "F.Cu") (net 1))
 (segment (start 150 90.5) (end 148.5 92) (width 0.25) (layer "F.Cu") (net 1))
 (segment (start 128 78) (end 130 80) (width 0.25) (layer "F.Cu") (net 1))
 (segment (start 130 80) (end 135 80) (width 0.25) (layer "F.Cu") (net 1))
 (segment (start 138.5 88.5) (end 134.5 88.5) (width 0.25) (layer "F.Cu") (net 1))
 (segment (start 148 63) (end 148 64.5) (width 0.25) (layer "F.Cu") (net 1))
 (segment (start 134.5 88.5) (end 133.901562 87.901562) (width 0.25) (layer "F.Cu") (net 1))
 (segment (start 148 63) (end 150.5 63) (width 0.25) (layer "F.Cu") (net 1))
 (segment (start 131.5 64.5) (end 132 64) (width 0.25) (layer "F.Cu") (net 1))
 (segment (start 158.275 70) (end 162 73.725) (width 0.25) (layer "F.Cu") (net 1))
 (segment (start 155 79.5) (end 155 72) (width 0.25) (layer "F.Cu") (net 1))
 (segment (start 141.5 58) (end 143.725 58) (width 0.25) (layer "F.Cu") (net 1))
 (segment (start 151.5 61.5) (end 155.5 61.5) (width 0.25) (layer "F.Cu") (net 1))
 (segment (start 131.5 67.5) (end 131.5 64.5) (width 0.25) (layer "F.Cu") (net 1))
 (segment (start 135 68.5) (end 132.5 68.5) (width 0.25) (layer "F.Cu") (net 1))
 (segment (start 157 70) (end 158.275 70) (width 0.25) (layer "F.Cu") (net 1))
 (segment (start 148.5 92) (end 146.5 92) (width 0.25) (layer "F.Cu") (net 1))
 (segment (start 155.5 61.5) (end 156.098439 62.098439) (width 0.25) (layer "F.Cu") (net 1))
 (segment (start 160 84.000001) (end 157.901562 86.098439) (width 0.25) (layer "F.Cu") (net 1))
 (segment (start 132.5 68.5) (end 131.5 67.5) (width 0.25) (layer "F.Cu") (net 1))
 (segment (start 160 82) (end 160 84.000001) (width 0.25) (layer "F.Cu") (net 1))
 (segment (start 148.5 86) (end 155 79.5) (width 0.25) (layer "F.Cu") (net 1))
 (segment (start 150.5 67.5) (end 150.5 65.5) (width 0.25) (layer "F.Cu") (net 1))
 (segment (start 141 62.5) (end 140.5 62) (width 0.25) (layer "F.Cu") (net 1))
 (segment (start 135 80) (end 141 86) (width 0.25) (layer "F.Cu") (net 1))
 (segment (start 155 72) (end 150.5 67.5) (width 0.25) (layer "F.Cu") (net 1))
 (segment (start 148.5 86) (end 150 87.5) (width 0.25) (layer "F.Cu") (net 1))
 (segment (start 140.5 59) (end 141.5 58) (width 0.25) (layer "F.Cu") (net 1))
 (segment (start 134 79) (end 132 79) (width 0.25) (layer "F.Cu") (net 2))
 (segment (start 135 78) (end 134 79) (width 0.25) (layer "F.Cu") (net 2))
 (segment (start 135 78) (end 135 77) (width 0.25) (layer "F.Cu") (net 2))
 (via (at 132 79) (size 0.8) (drill 0.4) (layers "F.Cu" "B.Cu") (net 2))
 (segment (start 129.5 75) (end 129.5 79) (width 0.25) (layer "B.Cu") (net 2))
 (segment (start 147 62.5) (end 145.46 64.04) (width 0.25) (layer "B.Cu") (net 2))
 (segment (start 155.5 86) (end 160 81.5) (width 0.25) (layer "B.Cu") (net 2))
 (segment (start 133.101974 63.101974) (end 132.898026 63.101974) (width 0.25) (layer "B.Cu") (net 2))
 (segment (start 145.23 92) (end 145.23 90.73) (width 0.25) (layer "B.Cu") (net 2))
 (segment (start 160 75) (end 160 68.5) (width 0.25) (layer "B.Cu") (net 2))
 (segment (start 129.5 81) (end 134.5 86) (width 0.25) (layer "B.Cu") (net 2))
 (segment (start 134.5 86) (end 133.496464 87.003536) (width 0.25) (layer "B.Cu") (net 2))
 (segment (start 139 90.5) (end 145 90.5) (width 0.25) (layer "B.Cu") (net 2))
 (segment (start 132 79) (end 129.5 79) (width 0.25) (layer "B.Cu") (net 2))
 (segment (start 160 81.5) (end 160 75) (width 0.25) (layer "B.Cu") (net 2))
 (segment (start 151 90.5) (end 155.5 86) (width 0.25) (layer "B.Cu") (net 2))
 (segment (start 162 74.995) (end 160.005 74.995) (width 0.25) (layer "B.Cu") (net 2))
 (segment (start 129.27 75.23) (end 129.5 75) (width 0.25) (layer "B.Cu") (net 2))
 (segment (start 160 68.5) (end 154 62.5) (width 0.25) (layer "B.Cu") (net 2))
 (segment (start 129.5 68.5) (end 129.5 75) (width 0.25) (layer "B.Cu") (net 2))
 (segment (start 155.5 86) (end 156.496465 86.996465) (width 0.25) (layer "B.Cu") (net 2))
 (segment (start 144.49 59.5) (end 138.5 59.5) (width 0.25) (layer "B.Cu") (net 2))
 (segment (start 129.5 79) (end 129.5 81) (width 0.25) (layer "B.Cu") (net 2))
 (segment (start 134.5 86) (end 139 90.5) (width 0.25) (layer "B.Cu") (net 2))
 (segment (start 156.496465 86.996465) (end 157.003536 86.996465) (width 0.25) (layer "B.Cu") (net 2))
 (segment (start 138.5 59.5) (end 134 64) (width 0.25) (layer "B.Cu") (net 2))
 (segment (start 134 64) (end 133.101974 63.101974) (width 0.25) (layer "B.Cu") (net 2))
 (segment (start 144.995 58) (end 144.995 58.995) (width 0.25) (layer "B.Cu") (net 2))
 (segment (start 156.5 65) (end 156.5 63.49293) (width 0.25) (layer "B.Cu") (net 2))
 (segment (start 156.5 63.49293) (end 156.996465 62.996465) (width 0.25) (layer "B.Cu") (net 2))
 (segment (start 133.496464 87.003536) (end 133.003536 87.003536) (width 0.25) (layer "B.Cu") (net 2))
 (segment (start 128 75.23) (end 129.27 75.23) (width 0.25) (layer "B.Cu") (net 2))
 (segment (start 145.46 64.04) (end 145.46 64.5) (width 0.25) (layer "B.Cu") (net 2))
 (segment (start 160.005 74.995) (end 160 75) (width 0.25) (layer "B.Cu") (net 2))
 (segment (start 134 64) (end 129.5 68.5) (width 0.25) (layer "B.Cu") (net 2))
 (segment (start 145.23 90.73) (end 145 90.5) (width 0.25) (layer "B.Cu") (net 2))
 (segment (start 145 90.5) (end 151 90.5) (width 0.25) (layer "B.Cu") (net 2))
 (segment (start 154 62.5) (end 147 62.5) (width 0.25) (layer "B.Cu") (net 2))
 (segment (start 144.995 58.995) (end 144.49 59.5) (width 0.25) (layer "B.Cu") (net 2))
 (segment (start 135 71) (end 135 73) (width 0.25) (layer "F.Cu") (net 12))
 (segment (start 136.819132 69.180868) (end 135 71) (width 0.25) (layer "F.Cu") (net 12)))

